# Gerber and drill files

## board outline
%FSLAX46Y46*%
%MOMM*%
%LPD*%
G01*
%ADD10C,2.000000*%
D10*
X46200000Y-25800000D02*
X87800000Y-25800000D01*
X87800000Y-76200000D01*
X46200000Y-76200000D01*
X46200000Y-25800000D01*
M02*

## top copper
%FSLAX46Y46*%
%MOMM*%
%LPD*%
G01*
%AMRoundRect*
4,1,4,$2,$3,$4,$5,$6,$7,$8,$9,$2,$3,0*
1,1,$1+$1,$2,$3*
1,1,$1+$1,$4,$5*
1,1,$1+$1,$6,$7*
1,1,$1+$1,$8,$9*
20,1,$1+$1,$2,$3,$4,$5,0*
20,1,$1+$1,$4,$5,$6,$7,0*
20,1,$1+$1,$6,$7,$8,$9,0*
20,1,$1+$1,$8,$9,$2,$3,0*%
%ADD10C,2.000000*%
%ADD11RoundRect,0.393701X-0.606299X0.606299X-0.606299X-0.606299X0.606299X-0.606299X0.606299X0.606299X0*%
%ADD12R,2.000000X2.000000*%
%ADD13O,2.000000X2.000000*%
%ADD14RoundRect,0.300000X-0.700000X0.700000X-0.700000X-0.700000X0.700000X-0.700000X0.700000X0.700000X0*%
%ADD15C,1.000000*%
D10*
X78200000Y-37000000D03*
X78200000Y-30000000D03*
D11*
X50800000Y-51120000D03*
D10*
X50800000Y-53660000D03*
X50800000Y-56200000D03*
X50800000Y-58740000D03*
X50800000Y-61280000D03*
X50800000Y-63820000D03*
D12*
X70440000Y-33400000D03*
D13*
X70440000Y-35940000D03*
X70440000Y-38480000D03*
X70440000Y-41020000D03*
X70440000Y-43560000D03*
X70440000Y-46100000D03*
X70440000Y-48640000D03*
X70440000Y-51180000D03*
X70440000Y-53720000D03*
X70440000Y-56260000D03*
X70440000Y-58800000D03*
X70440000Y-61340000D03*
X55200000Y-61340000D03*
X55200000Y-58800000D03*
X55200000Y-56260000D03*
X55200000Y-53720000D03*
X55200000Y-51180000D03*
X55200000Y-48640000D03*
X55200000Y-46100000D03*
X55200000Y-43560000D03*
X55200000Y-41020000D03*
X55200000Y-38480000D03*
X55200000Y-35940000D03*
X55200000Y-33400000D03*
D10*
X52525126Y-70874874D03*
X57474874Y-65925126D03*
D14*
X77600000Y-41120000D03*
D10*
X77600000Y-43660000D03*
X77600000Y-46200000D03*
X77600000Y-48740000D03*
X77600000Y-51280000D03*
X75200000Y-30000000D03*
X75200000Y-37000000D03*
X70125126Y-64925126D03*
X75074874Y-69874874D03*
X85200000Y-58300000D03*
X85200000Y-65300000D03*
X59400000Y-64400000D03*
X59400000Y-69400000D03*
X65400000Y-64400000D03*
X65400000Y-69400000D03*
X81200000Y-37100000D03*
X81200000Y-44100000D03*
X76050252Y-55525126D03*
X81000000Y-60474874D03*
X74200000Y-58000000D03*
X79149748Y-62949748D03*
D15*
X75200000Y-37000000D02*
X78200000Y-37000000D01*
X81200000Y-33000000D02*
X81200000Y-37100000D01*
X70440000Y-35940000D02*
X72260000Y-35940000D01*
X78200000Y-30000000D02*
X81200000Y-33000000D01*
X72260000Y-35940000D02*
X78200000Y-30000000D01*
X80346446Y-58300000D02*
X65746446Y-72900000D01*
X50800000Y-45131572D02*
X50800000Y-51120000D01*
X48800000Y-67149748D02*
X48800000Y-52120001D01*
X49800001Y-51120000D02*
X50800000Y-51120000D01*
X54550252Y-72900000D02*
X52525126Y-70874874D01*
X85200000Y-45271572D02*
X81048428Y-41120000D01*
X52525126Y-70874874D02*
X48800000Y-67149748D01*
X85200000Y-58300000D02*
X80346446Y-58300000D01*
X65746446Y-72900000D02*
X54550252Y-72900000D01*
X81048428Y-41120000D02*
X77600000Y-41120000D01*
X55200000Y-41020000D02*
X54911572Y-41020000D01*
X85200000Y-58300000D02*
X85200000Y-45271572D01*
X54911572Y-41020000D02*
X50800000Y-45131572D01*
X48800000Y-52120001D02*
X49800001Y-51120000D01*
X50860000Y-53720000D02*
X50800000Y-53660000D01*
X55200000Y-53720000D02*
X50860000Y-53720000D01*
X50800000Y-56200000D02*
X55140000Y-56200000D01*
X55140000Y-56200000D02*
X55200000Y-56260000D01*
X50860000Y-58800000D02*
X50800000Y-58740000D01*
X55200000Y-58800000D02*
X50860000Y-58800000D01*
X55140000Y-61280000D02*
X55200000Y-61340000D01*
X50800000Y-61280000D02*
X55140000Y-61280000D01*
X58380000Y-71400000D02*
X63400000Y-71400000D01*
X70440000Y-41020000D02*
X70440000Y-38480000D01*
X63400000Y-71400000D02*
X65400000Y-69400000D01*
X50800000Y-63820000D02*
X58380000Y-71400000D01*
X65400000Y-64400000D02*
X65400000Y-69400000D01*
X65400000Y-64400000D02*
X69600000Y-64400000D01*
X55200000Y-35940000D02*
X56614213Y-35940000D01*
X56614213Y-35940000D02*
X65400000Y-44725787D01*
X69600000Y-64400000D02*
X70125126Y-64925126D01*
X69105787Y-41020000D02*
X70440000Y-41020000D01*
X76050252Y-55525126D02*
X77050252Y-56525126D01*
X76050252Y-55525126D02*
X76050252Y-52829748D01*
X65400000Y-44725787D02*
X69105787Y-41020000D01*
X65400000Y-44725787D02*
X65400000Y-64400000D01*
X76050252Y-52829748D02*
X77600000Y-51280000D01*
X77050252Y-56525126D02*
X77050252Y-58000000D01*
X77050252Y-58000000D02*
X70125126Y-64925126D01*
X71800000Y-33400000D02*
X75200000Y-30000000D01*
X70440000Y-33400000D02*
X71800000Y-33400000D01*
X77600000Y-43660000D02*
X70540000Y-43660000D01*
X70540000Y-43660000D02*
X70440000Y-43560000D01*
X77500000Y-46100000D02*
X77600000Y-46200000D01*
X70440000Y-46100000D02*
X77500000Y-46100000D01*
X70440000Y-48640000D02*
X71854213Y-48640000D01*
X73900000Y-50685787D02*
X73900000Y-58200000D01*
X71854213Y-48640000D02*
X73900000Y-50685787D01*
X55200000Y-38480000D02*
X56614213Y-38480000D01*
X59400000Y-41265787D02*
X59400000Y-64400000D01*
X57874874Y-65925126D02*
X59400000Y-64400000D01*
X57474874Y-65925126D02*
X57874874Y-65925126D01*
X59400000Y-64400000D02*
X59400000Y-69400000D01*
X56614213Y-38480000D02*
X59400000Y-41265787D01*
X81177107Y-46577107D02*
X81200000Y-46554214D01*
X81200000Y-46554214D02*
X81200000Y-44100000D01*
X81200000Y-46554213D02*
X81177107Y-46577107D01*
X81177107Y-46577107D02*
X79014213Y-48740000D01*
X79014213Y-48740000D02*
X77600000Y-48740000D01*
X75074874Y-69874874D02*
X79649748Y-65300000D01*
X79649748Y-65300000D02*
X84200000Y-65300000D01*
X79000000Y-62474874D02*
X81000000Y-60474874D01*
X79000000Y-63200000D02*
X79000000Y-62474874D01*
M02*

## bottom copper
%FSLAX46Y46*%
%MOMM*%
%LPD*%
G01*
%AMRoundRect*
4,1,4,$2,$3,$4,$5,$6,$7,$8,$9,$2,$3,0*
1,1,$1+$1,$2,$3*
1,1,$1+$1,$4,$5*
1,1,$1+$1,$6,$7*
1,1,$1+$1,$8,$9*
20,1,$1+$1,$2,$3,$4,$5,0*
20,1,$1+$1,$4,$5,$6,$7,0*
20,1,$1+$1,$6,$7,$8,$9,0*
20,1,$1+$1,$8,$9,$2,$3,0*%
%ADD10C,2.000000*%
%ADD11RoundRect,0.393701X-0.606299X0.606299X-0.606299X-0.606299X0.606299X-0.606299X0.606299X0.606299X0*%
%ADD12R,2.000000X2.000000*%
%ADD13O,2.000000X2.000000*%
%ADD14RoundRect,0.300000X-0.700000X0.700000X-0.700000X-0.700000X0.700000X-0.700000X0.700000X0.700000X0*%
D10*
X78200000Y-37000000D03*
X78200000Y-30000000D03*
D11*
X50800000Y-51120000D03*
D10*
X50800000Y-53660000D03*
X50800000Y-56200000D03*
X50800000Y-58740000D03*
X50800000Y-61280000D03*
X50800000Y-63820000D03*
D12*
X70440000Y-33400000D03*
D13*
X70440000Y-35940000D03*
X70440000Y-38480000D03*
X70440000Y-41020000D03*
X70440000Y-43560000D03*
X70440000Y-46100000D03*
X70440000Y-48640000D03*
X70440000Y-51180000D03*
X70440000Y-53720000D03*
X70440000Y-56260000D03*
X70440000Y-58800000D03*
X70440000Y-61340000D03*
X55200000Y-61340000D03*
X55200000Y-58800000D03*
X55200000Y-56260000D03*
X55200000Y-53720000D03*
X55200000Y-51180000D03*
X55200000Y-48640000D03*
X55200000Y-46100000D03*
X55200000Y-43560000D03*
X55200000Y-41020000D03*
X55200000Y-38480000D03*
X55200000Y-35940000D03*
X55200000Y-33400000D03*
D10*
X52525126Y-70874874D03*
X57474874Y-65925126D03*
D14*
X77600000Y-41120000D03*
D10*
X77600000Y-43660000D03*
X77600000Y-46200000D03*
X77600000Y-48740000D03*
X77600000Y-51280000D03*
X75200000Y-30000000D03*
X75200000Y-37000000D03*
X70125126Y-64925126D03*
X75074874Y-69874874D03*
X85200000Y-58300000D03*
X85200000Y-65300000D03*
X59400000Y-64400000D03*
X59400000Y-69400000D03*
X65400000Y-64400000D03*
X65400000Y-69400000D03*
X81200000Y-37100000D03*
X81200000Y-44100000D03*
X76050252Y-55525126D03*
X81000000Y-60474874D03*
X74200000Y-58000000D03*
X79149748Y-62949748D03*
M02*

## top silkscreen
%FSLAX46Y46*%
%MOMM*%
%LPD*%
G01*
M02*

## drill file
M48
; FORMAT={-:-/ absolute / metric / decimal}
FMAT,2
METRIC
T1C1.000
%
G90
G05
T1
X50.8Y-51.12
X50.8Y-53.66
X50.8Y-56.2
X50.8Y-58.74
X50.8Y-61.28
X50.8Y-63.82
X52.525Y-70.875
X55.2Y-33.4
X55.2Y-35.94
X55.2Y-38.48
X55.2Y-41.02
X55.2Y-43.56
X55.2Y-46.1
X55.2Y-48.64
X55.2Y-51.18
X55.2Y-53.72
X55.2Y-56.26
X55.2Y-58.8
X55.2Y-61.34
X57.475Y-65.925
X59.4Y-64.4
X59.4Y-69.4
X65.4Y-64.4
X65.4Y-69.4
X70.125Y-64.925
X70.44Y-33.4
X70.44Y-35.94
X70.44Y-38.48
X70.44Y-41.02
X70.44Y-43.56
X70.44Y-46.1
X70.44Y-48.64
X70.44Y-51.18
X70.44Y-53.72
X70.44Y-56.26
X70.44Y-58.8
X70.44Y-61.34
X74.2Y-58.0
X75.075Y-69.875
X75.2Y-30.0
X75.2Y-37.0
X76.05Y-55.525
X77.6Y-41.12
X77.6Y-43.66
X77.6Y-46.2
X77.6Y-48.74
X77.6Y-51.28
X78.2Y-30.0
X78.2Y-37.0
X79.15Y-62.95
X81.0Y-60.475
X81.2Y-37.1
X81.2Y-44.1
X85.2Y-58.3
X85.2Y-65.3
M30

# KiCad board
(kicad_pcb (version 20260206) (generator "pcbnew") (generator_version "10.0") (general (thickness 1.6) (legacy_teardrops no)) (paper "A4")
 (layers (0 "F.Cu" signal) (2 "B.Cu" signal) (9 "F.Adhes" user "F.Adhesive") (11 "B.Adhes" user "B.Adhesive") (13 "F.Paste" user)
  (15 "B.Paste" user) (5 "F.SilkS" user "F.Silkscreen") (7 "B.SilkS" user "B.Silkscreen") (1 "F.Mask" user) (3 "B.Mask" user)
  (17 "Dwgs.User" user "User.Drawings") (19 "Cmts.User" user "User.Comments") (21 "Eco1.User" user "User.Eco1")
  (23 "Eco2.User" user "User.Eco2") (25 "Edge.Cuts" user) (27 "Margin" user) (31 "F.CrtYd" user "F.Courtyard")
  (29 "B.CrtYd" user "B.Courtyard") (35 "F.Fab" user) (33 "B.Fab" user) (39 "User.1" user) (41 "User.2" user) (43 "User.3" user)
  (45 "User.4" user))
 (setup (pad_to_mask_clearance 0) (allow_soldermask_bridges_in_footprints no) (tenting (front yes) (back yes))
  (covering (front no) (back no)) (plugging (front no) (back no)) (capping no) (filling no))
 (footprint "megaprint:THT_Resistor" (layer "B.Cu") (at 78.2 33.5 90)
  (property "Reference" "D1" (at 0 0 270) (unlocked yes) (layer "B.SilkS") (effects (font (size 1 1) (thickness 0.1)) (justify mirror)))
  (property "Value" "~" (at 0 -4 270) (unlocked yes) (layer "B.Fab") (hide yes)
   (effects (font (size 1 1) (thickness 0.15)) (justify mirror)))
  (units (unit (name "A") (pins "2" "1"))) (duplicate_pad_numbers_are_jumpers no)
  (pad "1" thru_hole circle (at -3.5 0 90) (size 2 2) (drill 1) (layers "*.Cu" "*.Mask") (remove_unused_layers no) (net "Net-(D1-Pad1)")
   (thermal_bridge_angle 90))
  (pad "2" thru_hole circle (at 3.5 0 90) (size 2 2) (drill 1) (layers "*.Cu" "*.Mask") (remove_unused_layers no) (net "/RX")
   (thermal_bridge_angle 90)))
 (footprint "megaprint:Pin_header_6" (layer "B.Cu") (at 50.8 57.4775 -90)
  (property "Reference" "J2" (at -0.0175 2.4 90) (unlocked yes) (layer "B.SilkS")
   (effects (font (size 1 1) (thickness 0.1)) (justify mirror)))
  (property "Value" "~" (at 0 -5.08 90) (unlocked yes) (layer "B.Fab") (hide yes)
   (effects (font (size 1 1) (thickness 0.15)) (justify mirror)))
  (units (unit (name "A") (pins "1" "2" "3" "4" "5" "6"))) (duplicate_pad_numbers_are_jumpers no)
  (pad "1" thru_hole roundrect (at -6.3575 0 270) (size 2 2) (drill 1) (layers "*.Cu" "*.Mask") (remove_unused_layers no)
   (roundrect_rratio 0.1968503937) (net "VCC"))
  (pad "2" thru_hole circle (at -3.8175 0 270) (size 2 2) (drill 1) (layers "*.Cu" "*.Mask") (remove_unused_layers no) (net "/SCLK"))
  (pad "3" thru_hole circle (at -1.2775 0 270) (size 2 2) (drill 1) (layers "*.Cu" "*.Mask") (remove_unused_layers no) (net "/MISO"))
  (pad "4" thru_hole circle (at 1.2625 0 270) (size 2 2) (drill 1) (layers "*.Cu" "*.Mask") (remove_unused_layers no) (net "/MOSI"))
  (pad "5" thru_hole circle (at 3.8025 0 270) (size 2 2) (drill 1) (layers "*.Cu" "*.Mask") (remove_unused_layers no) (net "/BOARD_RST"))
  (pad "6" thru_hole circle (at 6.3425 0 270) (size 2 2) (drill 1) (layers "*.Cu" "*.Mask") (remove_unused_layers no) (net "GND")))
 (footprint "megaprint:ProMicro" (layer "B.Cu") (at 62.82 44.83 180)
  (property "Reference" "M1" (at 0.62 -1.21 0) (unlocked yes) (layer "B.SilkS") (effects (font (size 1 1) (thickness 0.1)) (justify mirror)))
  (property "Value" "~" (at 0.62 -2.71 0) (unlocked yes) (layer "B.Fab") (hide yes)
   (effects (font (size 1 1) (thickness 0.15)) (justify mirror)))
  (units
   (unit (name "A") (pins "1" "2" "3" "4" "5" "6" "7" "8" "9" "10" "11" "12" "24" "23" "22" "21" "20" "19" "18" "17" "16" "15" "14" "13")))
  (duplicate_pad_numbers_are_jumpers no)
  (pad "1" thru_hole rect (at -7.62 11.43) (size 2 2) (drill 1) (layers "*.Cu" "*.Mask") (remove_unused_layers no) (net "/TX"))
  (pad "2" thru_hole oval (at -7.62 8.89) (size 2 2) (drill 1) (layers "*.Cu" "*.Mask") (remove_unused_layers no) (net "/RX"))
  (pad "3" thru_hole oval (at -7.62 6.35) (size 2 2) (drill 1) (layers "*.Cu" "*.Mask") (remove_unused_layers no) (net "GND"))
  (pad "4" thru_hole oval (at -7.62 3.81) (size 2 2) (drill 1) (layers "*.Cu" "*.Mask") (remove_unused_layers no) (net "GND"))
  (pad "5" thru_hole oval (at -7.62 1.27) (size 2 2) (drill 1) (layers "*.Cu" "*.Mask") (remove_unused_layers no) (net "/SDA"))
  (pad "6" thru_hole oval (at -7.62 -1.27) (size 2 2) (drill 1) (layers "*.Cu" "*.Mask") (remove_unused_layers no) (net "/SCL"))
  (pad "7" thru_hole oval (at -7.62 -3.81) (size 2 2) (drill 1) (layers "*.Cu" "*.Mask") (remove_unused_layers no) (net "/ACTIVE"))
  (pad "8" thru_hole oval (at -7.62 -6.35) (size 2 2) (drill 1) (layers "*.Cu" "*.Mask") (remove_unused_layers no)
   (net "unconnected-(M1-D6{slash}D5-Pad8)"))
  (pad "9" thru_hole oval (at -7.62 -8.89) (size 2 2) (drill 1) (layers "*.Cu" "*.Mask") (remove_unused_layers no)
   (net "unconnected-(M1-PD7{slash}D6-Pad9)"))
  (pad "10" thru_hole oval (at -7.62 -11.43) (size 2 2) (drill 1) (layers "*.Cu" "*.Mask") (remove_unused_layers no)
   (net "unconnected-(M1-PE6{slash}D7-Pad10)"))
  (pad "11" thru_hole oval (at -7.62 -13.97) (size 2 2) (drill 1) (layers "*.Cu" "*.Mask") (remove_unused_layers no)
   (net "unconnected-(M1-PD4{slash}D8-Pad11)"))
  (pad "12" thru_hole oval (at -7.62 -16.51) (size 2 2) (drill 1) (layers "*.Cu" "*.Mask") (remove_unused_layers no)
   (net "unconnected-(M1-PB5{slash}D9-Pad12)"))
  (pad "13" thru_hole oval (at 7.62 -16.51) (size 2 2) (drill 1) (layers "*.Cu" "*.Mask") (remove_unused_layers no) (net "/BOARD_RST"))
  (pad "14" thru_hole oval (at 7.62 -13.97) (size 2 2) (drill 1) (layers "*.Cu" "*.Mask") (remove_unused_layers no) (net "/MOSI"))
  (pad "15" thru_hole oval (at 7.62 -11.43) (size 2 2) (drill 1) (layers "*.Cu" "*.Mask") (remove_unused_layers no) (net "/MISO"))
  (pad "16" thru_hole oval (at 7.62 -8.89) (size 2 2) (drill 1) (layers "*.Cu" "*.Mask") (remove_unused_layers no) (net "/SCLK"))
  (pad "17" thru_hole oval (at 7.62 -6.35) (size 2 2) (drill 1) (layers "*.Cu" "*.Mask") (remove_unused_layers no)
   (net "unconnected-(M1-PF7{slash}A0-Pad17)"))
  (pad "18" thru_hole oval (at 7.62 -3.81) (size 2 2) (drill 1) (layers "*.Cu" "*.Mask") (remove_unused_layers no)
   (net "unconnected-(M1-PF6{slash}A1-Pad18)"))
  (pad "19" thru_hole oval (at 7.62 -1.27) (size 2 2) (drill 1) (layers "*.Cu" "*.Mask") (remove_unused_layers no)
   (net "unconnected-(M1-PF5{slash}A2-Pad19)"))
  (pad "20" thru_hole oval (at 7.62 1.27) (size 2 2) (drill 1) (layers "*.Cu" "*.Mask") (remove_unused_layers no)
   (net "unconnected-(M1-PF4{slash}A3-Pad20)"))
  (pad "21" thru_hole oval (at 7.62 3.81) (size 2 2) (drill 1) (layers "*.Cu" "*.Mask") (remove_unused_layers no) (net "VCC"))
  (pad "22" thru_hole oval (at 7.62 6.35) (size 2 2) (drill 1) (layers "*.Cu" "*.Mask") (remove_unused_layers no) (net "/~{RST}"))
  (pad "23" thru_hole oval (at 7.62 8.89) (size 2 2) (drill 1) (layers "*.Cu" "*.Mask") (remove_unused_layers no) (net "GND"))
  (pad "24" thru_hole oval (at 7.62 11.43) (size 2 2) (drill 1) (layers "*.Cu" "*.Mask") (remove_unused_layers no)
   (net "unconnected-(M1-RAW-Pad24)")))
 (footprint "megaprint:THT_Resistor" (layer "B.Cu") (at 55 68.4 45)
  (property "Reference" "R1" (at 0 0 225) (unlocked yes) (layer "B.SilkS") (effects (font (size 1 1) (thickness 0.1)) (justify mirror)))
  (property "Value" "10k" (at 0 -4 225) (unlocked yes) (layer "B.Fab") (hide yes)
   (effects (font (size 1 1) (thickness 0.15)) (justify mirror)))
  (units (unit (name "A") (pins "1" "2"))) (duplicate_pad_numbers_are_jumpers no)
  (pad "1" thru_hole circle (at -3.5 0 45) (size 2 2) (drill 1) (layers "*.Cu" "*.Mask") (remove_unused_layers no) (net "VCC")
   (thermal_bridge_angle 90))
  (pad "2" thru_hole circle (at 3.5 0 45) (size 2 2) (drill 1) (layers "*.Cu" "*.Mask") (remove_unused_layers no) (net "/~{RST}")
   (thermal_bridge_angle 90)))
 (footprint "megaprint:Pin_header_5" (layer "B.Cu") (at 77.6 46.2 -90)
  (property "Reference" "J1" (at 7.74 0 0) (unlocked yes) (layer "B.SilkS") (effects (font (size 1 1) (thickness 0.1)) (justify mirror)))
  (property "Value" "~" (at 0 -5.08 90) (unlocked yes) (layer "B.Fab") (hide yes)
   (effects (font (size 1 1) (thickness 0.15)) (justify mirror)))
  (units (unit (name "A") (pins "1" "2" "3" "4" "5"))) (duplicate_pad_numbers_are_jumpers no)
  (pad "1" thru_hole roundrect (at -5.08 0 270) (size 2 2) (drill 1) (layers "*.Cu" "*.Mask") (remove_unused_layers no)
   (roundrect_rratio 0.15) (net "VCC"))
  (pad "2" thru_hole circle (at -2.54 0 270) (size 2 2) (drill 1) (layers "*.Cu" "*.Mask") (remove_unused_layers no) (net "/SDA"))
  (pad "3" thru_hole circle (at 0 0 270) (size 2 2) (drill 1) (layers "*.Cu" "*.Mask") (remove_unused_layers no) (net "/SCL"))
  (pad "4" thru_hole circle (at 2.54 0 270) (size 2 2) (drill 1) (layers "*.Cu" "*.Mask") (remove_unused_layers no) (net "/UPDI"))
  (pad "5" thru_hole circle (at 5.08 0 270) (size 2 2) (drill 1) (layers "*.Cu" "*.Mask") (remove_unused_layers no) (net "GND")))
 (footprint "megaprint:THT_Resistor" (layer "B.Cu") (at 75.2 33.5 -90)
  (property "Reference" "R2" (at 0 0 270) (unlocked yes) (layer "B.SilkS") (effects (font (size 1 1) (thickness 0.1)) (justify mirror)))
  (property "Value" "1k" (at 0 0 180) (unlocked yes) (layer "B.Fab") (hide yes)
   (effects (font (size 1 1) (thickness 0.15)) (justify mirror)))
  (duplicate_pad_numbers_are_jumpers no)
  (pad "1" thru_hole circle (at -3.5 0 270) (size 2 2) (drill 1) (layers "*.Cu" "*.Mask") (remove_unused_layers no) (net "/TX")
   (thermal_bridge_angle 90))
  (pad "2" thru_hole circle (at 3.5 0 270) (size 2 2) (drill 1) (layers "*.Cu" "*.Mask") (remove_unused_layers no) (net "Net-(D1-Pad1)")
   (thermal_bridge_angle 90)))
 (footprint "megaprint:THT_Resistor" (layer "B.Cu") (at 72.6 67.4 -45)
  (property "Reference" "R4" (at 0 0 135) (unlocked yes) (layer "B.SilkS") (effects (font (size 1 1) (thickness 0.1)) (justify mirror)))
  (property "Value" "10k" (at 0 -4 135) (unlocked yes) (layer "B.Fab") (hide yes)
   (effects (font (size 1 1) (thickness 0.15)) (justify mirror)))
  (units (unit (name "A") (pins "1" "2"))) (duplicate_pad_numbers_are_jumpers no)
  (pad "1" thru_hole circle (at -3.5 0 315) (size 2 2) (drill 1) (layers "*.Cu" "*.Mask") (remove_unused_layers no) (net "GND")
   (thermal_bridge_angle 90))
  (pad "2" thru_hole circle (at 3.5 0 315) (size 2 2) (drill 1) (layers "*.Cu" "*.Mask") (remove_unused_layers no) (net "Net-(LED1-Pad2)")
   (thermal_bridge_angle 90)))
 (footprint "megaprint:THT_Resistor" (layer "B.Cu") (at 85.2 61.8 -90)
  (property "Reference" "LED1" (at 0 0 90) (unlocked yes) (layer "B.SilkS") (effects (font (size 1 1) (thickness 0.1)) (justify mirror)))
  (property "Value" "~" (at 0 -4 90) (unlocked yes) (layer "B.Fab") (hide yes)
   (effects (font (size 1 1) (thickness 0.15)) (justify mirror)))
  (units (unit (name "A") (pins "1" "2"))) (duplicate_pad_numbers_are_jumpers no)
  (pad "1" thru_hole circle (at -3.5 0 270) (size 2 2) (drill 1) (layers "*.Cu" "*.Mask") (remove_unused_layers no) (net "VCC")
   (thermal_bridge_angle 90))
  (pad "2" thru_hole circle (at 3.5 0 270) (size 2 2) (drill 1) (layers "*.Cu" "*.Mask") (remove_unused_layers no) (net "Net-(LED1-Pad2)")
   (thermal_bridge_angle 90)))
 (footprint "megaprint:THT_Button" (layer "B.Cu") (at 62.4 66.9)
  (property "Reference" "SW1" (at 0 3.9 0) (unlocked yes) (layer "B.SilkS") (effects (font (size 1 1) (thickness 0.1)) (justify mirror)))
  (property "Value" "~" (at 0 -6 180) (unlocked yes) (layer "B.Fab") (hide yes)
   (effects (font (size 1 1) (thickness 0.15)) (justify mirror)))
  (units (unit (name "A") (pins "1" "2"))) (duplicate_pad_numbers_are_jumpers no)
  (pad "1" thru_hole circle (at -3 -2.5 180) (size 2 2) (drill 1) (layers "*.Cu" "*.Mask") (remove_unused_layers no) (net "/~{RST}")
   (thermal_bridge_angle 90))
  (pad "1" thru_hole circle (at -3 2.5 180) (size 2 2) (drill 1) (layers "*.Cu" "*.Mask") (remove_unused_layers no) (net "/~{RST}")
   (thermal_bridge_angle 90))
  (pad "2" thru_hole circle (at 3 -2.5 180) (size 2 2) (drill 1) (layers "*.Cu" "*.Mask") (remove_unused_layers no) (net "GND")
   (thermal_bridge_angle 90))
  (pad "2" thru_hole circle (at 3 2.5 180) (size 2 2) (drill 1) (layers "*.Cu" "*.Mask") (remove_unused_layers no) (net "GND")
   (thermal_bridge_angle 90)))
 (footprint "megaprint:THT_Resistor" (layer "B.Cu") (at 81.2 40.6 -90)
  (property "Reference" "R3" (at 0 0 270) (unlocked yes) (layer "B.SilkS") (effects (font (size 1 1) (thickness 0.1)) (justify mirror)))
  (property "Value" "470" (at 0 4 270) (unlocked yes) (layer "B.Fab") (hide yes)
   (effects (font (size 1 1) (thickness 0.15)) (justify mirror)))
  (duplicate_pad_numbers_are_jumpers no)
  (pad "1" thru_hole circle (at -3.5 0 270) (size 2 2) (drill 1) (layers "*.Cu" "*.Mask") (remove_unused_layers no) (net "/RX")
   (thermal_bridge_angle 90))
  (pad "2" thru_hole circle (at 3.5 0 270) (size 2 2) (drill 1) (layers "*.Cu" "*.Mask") (remove_unused_layers no) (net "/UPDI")
   (thermal_bridge_angle 90)))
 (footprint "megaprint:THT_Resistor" (layer "B.Cu") (at 78.525126 58 -45)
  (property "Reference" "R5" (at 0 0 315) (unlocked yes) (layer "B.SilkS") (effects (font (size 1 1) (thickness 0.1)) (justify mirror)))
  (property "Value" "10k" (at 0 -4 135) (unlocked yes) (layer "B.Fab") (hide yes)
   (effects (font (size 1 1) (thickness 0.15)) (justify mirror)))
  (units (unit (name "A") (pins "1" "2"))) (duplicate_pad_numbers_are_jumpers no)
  (pad "1" thru_hole circle (at -3.5 0 315) (size 2 2) (drill 1) (layers "*.Cu" "*.Mask") (remove_unused_layers no) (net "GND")
   (thermal_bridge_angle 90))
  (pad "2" thru_hole circle (at 3.5 0 315) (size 2 2) (drill 1) (layers "*.Cu" "*.Mask") (remove_unused_layers no) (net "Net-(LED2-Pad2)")
   (thermal_bridge_angle 90)))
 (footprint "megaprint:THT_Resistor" (layer "B.Cu") (at 76.674874 60.474874 -45)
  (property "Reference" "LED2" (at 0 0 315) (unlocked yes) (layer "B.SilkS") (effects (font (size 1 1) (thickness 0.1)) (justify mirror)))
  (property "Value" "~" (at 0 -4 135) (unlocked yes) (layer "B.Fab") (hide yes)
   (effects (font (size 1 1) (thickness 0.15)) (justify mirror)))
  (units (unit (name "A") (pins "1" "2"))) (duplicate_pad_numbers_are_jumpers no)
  (pad "1" thru_hole circle (at -3.5 0 315) (size 2 2) (drill 1) (layers "*.Cu" "*.Mask") (remove_unused_layers no) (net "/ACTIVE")
   (thermal_bridge_angle 90))
  (pad "2" thru_hole circle (at 3.5 0 315) (size 2 2) (drill 1) (layers "*.Cu" "*.Mask") (remove_unused_layers no) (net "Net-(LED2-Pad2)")
   (thermal_bridge_angle 90)))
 (gr_rect (start 46.2 25.8) (end 87.8 76.2) (stroke (width 2) (type default)) (fill no) (layer "Edge.Cuts"))
 (segment (start 75.2 37) (end 78.2 37) (width 1) (layer "F.Cu") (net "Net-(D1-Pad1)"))
 (segment (start 81.2 33) (end 81.2 37.1) (width 1) (layer "F.Cu") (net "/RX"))
 (segment (start 70.44 35.94) (end 72.26 35.94) (width 1) (layer "F.Cu") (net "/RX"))
 (segment (start 78.2 30) (end 81.2 33) (width 1) (layer "F.Cu") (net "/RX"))
 (segment (start 72.26 35.94) (end 78.2 30) (width 1) (layer "F.Cu") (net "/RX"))
 (segment (start 80.346446 58.3) (end 65.746446 72.9) (width 1) (layer "F.Cu") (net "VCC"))
 (segment (start 50.8 45.131572) (end 50.8 51.12) (width 1) (layer "F.Cu") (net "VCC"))
 (segment (start 48.8 67.149748) (end 48.8 52.120001) (width 1) (layer "F.Cu") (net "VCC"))
 (segment (start 49.800001 51.12) (end 50.8 51.12) (width 1) (layer "F.Cu") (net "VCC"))
 (segment (start 54.550252 72.9) (end 52.525126 70.874874) (width 1) (layer "F.Cu") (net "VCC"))
 (segment (start 85.2 45.271572) (end 81.048428 41.12) (width 1) (layer "F.Cu") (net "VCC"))
 (segment (start 52.525126 70.874874) (end 48.8 67.149748) (width 1) (layer "F.Cu") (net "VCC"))
 (segment (start 85.2 58.3) (end 80.346446 58.3) (width 1) (layer "F.Cu") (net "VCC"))
 (segment (start 65.746446 72.9) (end 54.550252 72.9) (width 1) (layer "F.Cu") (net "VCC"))
 (segment (start 81.048428 41.12) (end 77.6 41.12) (width 1) (layer "F.Cu") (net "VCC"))
 (segment (start 55.2 41.02) (end 54.911572 41.02) (width 1) (layer "F.Cu") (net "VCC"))
 (segment (start 85.2 58.3) (end 85.2 45.271572) (width 1) (layer "F.Cu") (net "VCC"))
 (segment (start 54.911572 41.02) (end 50.8 45.131572) (width 1) (layer "F.Cu") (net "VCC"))
 (segment (start 48.8 52.120001) (end 49.800001 51.12) (width 1) (layer "F.Cu") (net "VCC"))
 (segment (start 50.86 53.72) (end 50.8 53.66) (width 1) (layer "F.Cu") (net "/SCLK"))
 (segment (start 55.2 53.72) (end 50.86 53.72) (width 1) (layer "F.Cu") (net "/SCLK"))
 (segment (start 50.8 56.2) (end 55.14 56.2) (width 1) (layer "F.Cu") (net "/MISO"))
 (segment (start 55.14 56.2) (end 55.2 56.26) (width 1) (layer "F.Cu") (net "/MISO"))
 (segment (start 50.86 58.8) (end 50.8 58.74) (width 1) (layer "F.Cu") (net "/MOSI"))
 (segment (start 55.2 58.8) (end 50.86 58.8) (width 1) (layer "F.Cu") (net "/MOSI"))
 (segment (start 55.14 61.28) (end 55.2 61.34) (width 1) (layer "F.Cu") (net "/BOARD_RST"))
 (segment (start 50.8 61.28) (end 55.14 61.28) (width 1) (layer "F.Cu") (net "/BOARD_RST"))
 (segment (start 58.38 71.4) (end 63.4 71.4) (width 1) (layer "F.Cu") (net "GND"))
 (segment (start 70.44 41.02) (end 70.44 38.48) (width 1) (layer "F.Cu") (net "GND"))
 (segment (start 63.4 71.4) (end 65.4 69.4) (width 1) (layer "F.Cu") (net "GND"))
 (segment (start 50.8 63.82) (end 58.38 71.4) (width 1) (layer "F.Cu") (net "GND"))
 (segment (start 65.4 64.4) (end 65.4 69.4) (width 1) (layer "F.Cu") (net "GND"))
 (segment (start 65.4 64.4) (end 69.6 64.4) (width 1) (layer "F.Cu") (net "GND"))
 (segment (start 55.2 35.94) (end 56.614213 35.94) (width 1) (layer "F.Cu") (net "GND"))
 (segment (start 56.614213 35.94) (end 65.4 44.725787) (width 1) (layer "F.Cu") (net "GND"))
 (segment (start 69.6 64.4) (end 70.125126 64.925126) (width 1) (layer "F.Cu") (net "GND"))
 (segment (start 69.105787 41.02) (end 70.44 41.02) (width 1) (layer "F.Cu") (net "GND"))
 (segment (start 76.050252 55.525126) (end 77.050252 56.525126) (width 1) (layer "F.Cu") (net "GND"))
 (segment (start 76.050252 55.525126) (end 76.050252 52.829748) (width 1) (layer "F.Cu") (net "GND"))
 (segment (start 65.4 44.725787) (end 69.105787 41.02) (width 1) (layer "F.Cu") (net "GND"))
 (segment (start 65.4 44.725787) (end 65.4 64.4) (width 1) (layer "F.Cu") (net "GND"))
 (segment (start 76.050252 52.829748) (end 77.6 51.28) (width 1) (layer "F.Cu") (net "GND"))
 (segment (start 77.050252 56.525126) (end 77.050252 58) (width 1) (layer "F.Cu") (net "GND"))
 (segment (start 77.050252 58) (end 70.125126 64.925126) (width 1) (layer "F.Cu") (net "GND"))
 (segment (start 71.8 33.4) (end 75.2 30) (width 1) (layer "F.Cu") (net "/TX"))
 (segment (start 70.44 33.4) (end 71.8 33.4) (width 1) (layer "F.Cu") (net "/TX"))
 (segment (start 77.6 43.66) (end 70.54 43.66) (width 1) (layer "F.Cu") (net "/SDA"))
 (segment (start 70.54 43.66) (end 70.44 43.56) (width 1) (layer "F.Cu") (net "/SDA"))
 (segment (start 77.5 46.1) (end 77.6 46.2) (width 1) (layer "F.Cu") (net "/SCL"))
 (segment (start 70.44 46.1) (end 77.5 46.1) (width 1) (layer "F.Cu") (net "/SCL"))
 (segment (start 70.44 48.64) (end 71.854213 48.64) (width 1) (layer "F.Cu") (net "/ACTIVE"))
 (segment (start 73.9 50.685787) (end 73.9 58.2) (width 1) (layer "F.Cu") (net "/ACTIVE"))
 (segment (start 71.854213 48.64) (end 73.9 50.685787) (width 1) (layer "F.Cu") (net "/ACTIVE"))
 (segment (start 55.2 38.48) (end 56.614213 38.48) (width 1) (layer "F.Cu") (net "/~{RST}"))
 (segment (start 59.4 41.265787) (end 59.4 64.4) (width 1) (layer "F.Cu") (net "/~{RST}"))
 (segment (start 57.874874 65.925126) (end 59.4 64.4) (width 1) (layer "F.Cu") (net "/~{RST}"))
 (segment (start 57.474874 65.925126) (end 57.874874 65.925126) (width 1) (layer "F.Cu") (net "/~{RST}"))
 (segment (start 59.4 64.4) (end 59.4 69.4) (width 1) (layer "F.Cu") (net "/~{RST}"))
 (segment (start 56.614213 38.48) (end 59.4 41.265787) (width 1) (layer "F.Cu") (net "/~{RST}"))
 (segment (start 81.177107 46.577107) (end 81.2 46.554214) (width 1) (layer "F.Cu") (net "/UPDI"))
 (segment (start 81.2 46.554214) (end 81.2 44.1) (width 1) (layer "F.Cu") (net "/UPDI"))
 (segment (start 81.2 46.554213) (end 81.177107 46.577107) (width 1) (layer "F.Cu") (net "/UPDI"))
 (segment (start 81.177107 46.577107) (end 79.014213 48.74) (width 1) (layer "F.Cu") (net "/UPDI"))
 (segment (start 79.014213 48.74) (end 77.6 48.74) (width 1) (layer "F.Cu") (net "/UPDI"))
 (segment (start 75.074874 69.874874) (end 79.649748 65.3) (width 1) (layer "F.Cu") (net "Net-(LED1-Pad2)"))
 (segment (start 79.649748 65.3) (end 84.2 65.3) (width 1) (layer "F.Cu") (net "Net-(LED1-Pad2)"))
 (segment (start 79 62.474874) (end 81 60.474874) (width 1) (layer "F.Cu") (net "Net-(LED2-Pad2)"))
 (segment (start 79 63.2) (end 79 62.474874) (width 1) (layer "F.Cu") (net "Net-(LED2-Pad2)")))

